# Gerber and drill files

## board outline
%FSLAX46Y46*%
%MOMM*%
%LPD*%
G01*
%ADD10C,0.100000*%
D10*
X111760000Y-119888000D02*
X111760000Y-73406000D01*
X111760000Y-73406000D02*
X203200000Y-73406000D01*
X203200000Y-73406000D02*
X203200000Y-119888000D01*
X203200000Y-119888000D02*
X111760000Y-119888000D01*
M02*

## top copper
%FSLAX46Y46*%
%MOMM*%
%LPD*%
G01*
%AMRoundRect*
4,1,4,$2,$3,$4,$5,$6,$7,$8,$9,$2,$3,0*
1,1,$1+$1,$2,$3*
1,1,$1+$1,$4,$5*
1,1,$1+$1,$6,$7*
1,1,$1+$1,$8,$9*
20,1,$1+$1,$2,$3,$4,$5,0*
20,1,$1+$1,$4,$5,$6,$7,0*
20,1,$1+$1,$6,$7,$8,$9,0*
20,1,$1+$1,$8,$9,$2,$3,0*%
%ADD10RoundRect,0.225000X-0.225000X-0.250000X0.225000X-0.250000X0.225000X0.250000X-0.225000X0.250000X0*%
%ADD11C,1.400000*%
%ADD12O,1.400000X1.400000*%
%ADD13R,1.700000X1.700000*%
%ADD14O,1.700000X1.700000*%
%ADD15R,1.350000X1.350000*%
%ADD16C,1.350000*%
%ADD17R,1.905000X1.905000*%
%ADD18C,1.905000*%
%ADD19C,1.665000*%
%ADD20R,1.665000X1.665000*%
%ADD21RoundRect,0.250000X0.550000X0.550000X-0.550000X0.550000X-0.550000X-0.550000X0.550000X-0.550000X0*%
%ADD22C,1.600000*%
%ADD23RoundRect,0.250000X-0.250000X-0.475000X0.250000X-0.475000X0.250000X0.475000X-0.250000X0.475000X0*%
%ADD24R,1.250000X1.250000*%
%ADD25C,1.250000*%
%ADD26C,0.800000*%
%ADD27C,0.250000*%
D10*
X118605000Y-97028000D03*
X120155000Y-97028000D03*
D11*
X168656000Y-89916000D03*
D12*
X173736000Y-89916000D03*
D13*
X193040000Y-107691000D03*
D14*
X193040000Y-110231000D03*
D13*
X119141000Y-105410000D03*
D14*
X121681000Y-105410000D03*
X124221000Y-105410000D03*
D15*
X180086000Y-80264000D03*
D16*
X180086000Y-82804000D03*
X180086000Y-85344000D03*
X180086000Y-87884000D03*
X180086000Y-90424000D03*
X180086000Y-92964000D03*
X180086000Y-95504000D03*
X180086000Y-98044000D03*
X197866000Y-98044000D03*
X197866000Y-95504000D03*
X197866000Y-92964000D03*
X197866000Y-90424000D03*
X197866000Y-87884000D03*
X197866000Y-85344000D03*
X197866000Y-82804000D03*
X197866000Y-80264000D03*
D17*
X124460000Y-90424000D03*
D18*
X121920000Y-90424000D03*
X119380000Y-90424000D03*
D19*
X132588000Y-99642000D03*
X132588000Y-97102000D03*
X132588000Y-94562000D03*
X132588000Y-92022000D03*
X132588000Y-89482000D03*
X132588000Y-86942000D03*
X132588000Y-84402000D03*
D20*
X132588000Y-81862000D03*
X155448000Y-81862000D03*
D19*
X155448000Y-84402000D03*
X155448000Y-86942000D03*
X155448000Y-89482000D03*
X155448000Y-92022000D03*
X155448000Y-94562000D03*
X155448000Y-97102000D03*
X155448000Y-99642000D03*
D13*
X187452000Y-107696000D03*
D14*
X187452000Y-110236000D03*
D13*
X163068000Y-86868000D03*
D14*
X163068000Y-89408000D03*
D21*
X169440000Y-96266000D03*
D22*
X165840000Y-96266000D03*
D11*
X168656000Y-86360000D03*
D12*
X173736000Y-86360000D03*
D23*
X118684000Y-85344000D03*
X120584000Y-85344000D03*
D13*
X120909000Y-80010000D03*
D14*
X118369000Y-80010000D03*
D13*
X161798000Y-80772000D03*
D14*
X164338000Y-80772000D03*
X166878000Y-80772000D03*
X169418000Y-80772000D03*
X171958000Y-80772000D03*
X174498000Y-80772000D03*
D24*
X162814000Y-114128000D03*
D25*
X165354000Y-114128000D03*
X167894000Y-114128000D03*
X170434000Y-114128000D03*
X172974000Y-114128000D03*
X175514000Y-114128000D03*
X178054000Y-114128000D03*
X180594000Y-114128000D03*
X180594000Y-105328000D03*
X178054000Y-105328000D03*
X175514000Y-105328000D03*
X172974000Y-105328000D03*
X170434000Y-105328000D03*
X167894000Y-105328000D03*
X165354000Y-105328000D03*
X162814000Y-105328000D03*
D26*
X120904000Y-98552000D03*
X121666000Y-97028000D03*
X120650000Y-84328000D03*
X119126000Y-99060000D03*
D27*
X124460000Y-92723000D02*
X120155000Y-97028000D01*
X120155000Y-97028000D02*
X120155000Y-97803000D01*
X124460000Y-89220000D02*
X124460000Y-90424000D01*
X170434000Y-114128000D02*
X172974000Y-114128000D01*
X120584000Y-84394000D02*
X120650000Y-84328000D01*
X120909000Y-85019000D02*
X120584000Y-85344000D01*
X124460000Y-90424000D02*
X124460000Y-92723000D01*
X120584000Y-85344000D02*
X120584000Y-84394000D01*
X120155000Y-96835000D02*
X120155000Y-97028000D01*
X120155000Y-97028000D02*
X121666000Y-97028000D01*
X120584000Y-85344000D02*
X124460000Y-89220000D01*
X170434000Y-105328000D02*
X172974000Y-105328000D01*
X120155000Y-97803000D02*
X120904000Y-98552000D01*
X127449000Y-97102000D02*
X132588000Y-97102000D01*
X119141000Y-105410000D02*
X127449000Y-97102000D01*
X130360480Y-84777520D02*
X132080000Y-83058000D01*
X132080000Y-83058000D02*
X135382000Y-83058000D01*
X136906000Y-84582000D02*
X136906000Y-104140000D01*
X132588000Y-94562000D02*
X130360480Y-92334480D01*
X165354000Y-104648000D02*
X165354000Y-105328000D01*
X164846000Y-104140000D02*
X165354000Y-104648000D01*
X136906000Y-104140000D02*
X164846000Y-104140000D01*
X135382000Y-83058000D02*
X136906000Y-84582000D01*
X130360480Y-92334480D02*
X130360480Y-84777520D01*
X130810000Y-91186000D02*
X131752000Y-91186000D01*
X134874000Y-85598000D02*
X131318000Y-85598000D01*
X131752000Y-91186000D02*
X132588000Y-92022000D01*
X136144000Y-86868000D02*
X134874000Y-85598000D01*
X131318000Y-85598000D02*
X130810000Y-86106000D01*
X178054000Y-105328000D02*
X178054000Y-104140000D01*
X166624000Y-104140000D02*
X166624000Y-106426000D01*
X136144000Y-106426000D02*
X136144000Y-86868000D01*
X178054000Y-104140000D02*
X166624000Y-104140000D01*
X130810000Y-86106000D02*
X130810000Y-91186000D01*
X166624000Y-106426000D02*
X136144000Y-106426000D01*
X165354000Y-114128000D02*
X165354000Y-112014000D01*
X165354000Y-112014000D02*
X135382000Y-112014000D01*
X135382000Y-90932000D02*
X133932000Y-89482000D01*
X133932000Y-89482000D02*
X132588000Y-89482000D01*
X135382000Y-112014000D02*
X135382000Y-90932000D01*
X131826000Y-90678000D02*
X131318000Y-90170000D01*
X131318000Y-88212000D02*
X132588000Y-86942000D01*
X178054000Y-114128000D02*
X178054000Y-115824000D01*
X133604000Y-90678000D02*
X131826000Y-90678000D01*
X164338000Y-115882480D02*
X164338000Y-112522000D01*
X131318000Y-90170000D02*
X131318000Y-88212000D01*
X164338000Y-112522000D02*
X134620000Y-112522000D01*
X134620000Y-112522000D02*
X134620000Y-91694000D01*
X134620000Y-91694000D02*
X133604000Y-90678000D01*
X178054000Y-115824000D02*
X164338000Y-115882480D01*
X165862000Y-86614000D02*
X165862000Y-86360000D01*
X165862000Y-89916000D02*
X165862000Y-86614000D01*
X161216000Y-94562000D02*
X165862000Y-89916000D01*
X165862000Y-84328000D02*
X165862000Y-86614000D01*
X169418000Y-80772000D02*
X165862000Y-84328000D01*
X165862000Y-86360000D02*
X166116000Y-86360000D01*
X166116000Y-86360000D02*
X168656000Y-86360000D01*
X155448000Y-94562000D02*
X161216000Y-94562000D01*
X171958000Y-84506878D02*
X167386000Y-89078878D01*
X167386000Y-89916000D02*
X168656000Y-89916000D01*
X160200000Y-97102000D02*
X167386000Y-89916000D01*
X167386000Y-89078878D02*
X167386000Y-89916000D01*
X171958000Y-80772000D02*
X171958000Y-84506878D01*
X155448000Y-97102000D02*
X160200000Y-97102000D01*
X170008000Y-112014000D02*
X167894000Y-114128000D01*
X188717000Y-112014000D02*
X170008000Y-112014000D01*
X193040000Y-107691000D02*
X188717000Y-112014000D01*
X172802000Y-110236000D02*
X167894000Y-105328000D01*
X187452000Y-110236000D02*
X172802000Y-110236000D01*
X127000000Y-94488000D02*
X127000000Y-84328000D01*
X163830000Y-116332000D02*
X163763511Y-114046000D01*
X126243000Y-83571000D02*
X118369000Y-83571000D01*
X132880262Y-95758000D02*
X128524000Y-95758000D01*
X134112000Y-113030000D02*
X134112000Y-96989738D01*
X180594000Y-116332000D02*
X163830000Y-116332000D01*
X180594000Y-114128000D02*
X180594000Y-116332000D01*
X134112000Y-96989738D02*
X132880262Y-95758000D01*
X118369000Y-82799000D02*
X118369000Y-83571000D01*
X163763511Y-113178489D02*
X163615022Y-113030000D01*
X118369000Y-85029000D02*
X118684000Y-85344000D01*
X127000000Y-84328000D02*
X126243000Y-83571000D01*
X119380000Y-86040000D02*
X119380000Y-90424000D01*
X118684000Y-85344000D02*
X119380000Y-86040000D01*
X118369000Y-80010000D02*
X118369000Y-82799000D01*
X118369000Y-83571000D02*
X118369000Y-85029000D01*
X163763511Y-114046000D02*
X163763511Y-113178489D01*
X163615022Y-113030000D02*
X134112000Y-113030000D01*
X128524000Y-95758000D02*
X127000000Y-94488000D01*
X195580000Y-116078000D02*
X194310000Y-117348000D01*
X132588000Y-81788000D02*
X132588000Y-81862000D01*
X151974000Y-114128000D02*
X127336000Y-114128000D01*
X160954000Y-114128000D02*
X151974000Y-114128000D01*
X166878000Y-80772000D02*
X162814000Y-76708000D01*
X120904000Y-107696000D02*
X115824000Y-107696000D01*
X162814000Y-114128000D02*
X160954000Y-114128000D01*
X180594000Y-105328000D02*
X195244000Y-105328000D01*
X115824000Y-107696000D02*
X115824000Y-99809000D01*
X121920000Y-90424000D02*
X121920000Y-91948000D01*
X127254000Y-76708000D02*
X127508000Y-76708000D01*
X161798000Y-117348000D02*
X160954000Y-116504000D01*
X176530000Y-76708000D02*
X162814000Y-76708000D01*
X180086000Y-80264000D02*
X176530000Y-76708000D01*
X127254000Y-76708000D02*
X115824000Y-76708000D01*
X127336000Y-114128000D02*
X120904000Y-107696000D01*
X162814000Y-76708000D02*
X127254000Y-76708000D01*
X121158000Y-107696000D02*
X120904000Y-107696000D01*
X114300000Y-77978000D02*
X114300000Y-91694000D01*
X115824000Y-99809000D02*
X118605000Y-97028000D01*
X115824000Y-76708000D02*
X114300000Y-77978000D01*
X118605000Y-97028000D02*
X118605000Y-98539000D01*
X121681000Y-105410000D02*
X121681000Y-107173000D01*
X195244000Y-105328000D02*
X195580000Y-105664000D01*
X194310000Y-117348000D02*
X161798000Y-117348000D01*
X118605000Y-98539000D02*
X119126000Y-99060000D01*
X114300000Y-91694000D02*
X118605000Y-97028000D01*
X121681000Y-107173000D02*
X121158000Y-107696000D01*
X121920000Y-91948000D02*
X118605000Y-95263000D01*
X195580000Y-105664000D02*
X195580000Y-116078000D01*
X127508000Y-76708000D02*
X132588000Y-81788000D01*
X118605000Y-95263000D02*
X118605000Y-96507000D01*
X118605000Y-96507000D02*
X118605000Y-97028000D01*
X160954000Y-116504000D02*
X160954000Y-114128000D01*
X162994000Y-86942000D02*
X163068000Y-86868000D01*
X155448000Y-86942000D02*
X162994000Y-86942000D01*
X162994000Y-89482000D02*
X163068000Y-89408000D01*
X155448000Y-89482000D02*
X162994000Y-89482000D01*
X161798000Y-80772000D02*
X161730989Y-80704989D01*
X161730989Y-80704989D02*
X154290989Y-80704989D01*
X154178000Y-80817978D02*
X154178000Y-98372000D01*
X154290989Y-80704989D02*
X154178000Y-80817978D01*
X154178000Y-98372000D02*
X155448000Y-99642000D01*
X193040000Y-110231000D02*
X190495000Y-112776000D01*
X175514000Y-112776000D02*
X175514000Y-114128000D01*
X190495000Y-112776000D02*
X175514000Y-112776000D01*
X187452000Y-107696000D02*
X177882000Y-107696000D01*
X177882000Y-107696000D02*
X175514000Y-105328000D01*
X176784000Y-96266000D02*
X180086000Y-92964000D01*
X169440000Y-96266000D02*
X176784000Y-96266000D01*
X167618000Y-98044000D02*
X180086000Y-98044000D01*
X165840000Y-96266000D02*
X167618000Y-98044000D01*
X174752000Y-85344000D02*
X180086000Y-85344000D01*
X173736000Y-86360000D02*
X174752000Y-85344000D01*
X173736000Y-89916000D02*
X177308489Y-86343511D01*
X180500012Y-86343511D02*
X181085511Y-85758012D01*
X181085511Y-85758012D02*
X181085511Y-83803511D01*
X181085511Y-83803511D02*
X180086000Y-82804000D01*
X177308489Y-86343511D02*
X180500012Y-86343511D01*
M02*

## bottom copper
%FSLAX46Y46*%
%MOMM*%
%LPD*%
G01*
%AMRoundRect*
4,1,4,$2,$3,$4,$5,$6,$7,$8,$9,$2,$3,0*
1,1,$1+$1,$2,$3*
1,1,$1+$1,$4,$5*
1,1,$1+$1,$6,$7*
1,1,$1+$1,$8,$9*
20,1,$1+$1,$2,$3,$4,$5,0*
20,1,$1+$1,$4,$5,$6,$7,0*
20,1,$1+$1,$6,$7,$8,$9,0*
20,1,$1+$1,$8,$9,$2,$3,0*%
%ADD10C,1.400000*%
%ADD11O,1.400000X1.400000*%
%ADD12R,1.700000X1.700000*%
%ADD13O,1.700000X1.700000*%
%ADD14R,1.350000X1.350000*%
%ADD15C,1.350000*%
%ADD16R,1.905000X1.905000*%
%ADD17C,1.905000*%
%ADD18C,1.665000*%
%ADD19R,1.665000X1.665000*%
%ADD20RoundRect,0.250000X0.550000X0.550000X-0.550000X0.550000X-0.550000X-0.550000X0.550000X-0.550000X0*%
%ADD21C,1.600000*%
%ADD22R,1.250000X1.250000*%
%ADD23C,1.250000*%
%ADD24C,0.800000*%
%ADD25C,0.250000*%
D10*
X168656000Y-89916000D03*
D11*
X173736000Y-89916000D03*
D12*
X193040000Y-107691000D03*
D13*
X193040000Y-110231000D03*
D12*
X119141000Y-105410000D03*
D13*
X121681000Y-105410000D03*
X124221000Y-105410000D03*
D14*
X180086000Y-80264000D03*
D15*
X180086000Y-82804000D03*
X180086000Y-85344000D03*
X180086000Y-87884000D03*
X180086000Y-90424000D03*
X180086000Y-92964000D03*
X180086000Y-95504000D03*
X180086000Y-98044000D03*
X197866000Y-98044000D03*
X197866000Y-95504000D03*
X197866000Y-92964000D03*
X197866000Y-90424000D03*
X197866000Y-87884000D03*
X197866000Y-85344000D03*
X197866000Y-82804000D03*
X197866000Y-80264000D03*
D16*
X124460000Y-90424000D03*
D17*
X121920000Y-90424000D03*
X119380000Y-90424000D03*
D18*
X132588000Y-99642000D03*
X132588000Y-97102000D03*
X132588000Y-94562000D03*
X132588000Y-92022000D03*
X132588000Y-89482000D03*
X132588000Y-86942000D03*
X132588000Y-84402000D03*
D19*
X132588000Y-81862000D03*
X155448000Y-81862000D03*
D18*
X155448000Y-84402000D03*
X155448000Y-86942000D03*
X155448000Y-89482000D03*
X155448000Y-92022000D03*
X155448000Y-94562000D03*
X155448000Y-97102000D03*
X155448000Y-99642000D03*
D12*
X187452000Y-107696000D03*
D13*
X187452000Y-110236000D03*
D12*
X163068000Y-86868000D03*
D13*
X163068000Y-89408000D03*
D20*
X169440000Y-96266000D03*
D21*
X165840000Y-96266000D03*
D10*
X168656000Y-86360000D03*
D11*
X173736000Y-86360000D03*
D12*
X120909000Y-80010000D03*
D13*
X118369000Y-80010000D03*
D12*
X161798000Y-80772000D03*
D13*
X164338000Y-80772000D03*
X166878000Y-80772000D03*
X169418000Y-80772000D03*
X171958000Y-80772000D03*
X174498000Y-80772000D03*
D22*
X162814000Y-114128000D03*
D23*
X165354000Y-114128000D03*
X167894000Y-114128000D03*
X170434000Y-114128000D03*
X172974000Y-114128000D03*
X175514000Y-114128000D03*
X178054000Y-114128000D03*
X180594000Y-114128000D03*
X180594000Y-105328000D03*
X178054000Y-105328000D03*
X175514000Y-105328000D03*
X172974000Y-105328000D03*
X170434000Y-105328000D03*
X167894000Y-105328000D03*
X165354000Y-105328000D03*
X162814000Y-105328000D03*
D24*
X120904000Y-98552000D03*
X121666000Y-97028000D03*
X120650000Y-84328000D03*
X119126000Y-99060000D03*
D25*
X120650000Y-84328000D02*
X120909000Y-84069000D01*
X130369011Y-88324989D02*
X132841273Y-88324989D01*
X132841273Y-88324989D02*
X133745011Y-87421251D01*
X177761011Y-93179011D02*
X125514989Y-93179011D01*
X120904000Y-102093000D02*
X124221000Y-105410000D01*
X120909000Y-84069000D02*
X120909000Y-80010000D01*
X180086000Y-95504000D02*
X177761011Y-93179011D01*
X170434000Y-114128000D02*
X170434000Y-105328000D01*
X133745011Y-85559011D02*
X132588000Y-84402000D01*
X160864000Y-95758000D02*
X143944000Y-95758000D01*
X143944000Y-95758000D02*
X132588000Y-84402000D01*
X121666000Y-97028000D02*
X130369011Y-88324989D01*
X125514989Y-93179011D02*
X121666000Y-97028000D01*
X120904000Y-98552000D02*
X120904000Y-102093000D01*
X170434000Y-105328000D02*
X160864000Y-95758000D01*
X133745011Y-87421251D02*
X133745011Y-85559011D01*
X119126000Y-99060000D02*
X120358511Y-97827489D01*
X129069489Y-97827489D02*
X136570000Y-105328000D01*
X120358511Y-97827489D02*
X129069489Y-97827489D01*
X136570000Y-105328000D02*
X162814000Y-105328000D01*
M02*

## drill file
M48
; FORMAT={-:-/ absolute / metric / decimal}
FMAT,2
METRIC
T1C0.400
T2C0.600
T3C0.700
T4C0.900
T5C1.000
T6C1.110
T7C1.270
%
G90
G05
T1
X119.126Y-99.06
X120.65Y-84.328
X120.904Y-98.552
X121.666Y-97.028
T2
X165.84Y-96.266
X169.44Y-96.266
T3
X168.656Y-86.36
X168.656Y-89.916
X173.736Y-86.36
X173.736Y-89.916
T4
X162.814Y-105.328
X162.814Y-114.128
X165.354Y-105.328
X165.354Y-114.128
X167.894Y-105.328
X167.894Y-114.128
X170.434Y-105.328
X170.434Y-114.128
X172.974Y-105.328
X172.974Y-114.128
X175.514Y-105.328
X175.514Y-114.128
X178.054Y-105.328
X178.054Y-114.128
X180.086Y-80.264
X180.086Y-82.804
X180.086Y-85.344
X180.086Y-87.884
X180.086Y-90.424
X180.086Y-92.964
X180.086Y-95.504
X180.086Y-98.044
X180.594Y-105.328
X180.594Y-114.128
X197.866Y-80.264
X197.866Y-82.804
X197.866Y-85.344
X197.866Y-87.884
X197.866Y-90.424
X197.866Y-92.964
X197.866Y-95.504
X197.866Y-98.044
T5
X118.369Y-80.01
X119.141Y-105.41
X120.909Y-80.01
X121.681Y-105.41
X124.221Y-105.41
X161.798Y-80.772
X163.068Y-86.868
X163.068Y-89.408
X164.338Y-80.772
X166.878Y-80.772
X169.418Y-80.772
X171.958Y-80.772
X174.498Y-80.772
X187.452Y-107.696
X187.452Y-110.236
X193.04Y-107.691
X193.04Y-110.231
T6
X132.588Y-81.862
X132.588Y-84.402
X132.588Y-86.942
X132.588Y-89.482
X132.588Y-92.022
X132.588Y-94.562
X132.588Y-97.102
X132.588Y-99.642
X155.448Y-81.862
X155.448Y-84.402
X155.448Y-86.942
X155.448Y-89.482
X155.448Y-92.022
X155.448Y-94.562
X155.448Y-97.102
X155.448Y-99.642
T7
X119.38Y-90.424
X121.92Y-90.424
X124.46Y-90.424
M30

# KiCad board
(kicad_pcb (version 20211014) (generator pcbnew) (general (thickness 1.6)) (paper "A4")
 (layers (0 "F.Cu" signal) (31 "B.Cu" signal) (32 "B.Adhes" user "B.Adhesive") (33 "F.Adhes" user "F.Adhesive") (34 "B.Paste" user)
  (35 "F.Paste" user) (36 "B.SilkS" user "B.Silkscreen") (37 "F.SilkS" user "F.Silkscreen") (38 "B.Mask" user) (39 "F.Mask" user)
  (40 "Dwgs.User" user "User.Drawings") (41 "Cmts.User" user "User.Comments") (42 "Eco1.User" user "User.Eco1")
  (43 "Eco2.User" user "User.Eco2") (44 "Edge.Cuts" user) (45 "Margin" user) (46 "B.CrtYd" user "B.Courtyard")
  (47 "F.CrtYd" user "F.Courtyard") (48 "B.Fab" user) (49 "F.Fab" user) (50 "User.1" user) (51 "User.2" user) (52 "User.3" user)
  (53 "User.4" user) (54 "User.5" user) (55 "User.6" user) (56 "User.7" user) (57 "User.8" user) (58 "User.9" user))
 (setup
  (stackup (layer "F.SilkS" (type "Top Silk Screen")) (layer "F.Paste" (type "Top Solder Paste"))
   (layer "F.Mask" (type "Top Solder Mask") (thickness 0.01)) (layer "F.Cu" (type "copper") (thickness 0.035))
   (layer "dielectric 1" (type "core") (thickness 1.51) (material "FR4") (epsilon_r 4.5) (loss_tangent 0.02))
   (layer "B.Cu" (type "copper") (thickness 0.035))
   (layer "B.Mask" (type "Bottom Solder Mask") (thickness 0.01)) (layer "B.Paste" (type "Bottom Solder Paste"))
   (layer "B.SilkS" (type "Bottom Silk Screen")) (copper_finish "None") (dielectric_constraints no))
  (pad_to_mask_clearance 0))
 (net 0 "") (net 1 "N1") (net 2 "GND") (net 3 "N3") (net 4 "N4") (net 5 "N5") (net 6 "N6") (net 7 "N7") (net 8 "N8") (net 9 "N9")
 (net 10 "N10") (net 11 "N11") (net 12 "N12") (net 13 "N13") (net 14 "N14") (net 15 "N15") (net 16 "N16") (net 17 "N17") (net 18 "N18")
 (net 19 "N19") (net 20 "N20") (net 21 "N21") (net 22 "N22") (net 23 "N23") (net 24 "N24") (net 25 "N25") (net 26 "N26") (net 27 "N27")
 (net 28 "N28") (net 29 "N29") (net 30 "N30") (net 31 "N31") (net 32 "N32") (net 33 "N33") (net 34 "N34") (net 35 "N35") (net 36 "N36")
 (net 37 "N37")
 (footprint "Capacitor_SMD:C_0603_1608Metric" (layer "F.Cu") (at 119.38 97.028)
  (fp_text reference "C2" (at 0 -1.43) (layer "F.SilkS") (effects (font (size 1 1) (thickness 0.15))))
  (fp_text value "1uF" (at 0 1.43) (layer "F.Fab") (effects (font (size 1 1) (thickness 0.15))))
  (pad "1" smd roundrect locked (at -0.775 0) (size 0.9 0.95) (layers "F.Cu" "F.Paste" "F.Mask") (roundrect_rratio 0.25) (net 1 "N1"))
  (pad "2" smd roundrect locked (at 0.775 0) (size 0.9 0.95) (layers "F.Cu" "F.Paste" "F.Mask") (roundrect_rratio 0.25) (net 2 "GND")))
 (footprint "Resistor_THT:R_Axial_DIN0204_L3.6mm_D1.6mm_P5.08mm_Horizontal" (layer "F.Cu") (at 168.656 89.916)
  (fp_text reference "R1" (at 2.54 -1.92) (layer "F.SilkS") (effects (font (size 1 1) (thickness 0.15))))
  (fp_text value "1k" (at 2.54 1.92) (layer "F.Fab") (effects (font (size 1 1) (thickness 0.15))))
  (pad "1" thru_hole circle locked (at 0 0) (size 1.4 1.4) (drill 0.7) (layers *.Cu *.Mask) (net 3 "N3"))
  (pad "2" thru_hole oval locked (at 5.08 0) (size 1.4 1.4) (drill 0.7) (layers *.Cu *.Mask) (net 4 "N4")))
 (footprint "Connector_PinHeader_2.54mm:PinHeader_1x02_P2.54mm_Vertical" (layer "F.Cu") (at 193.04 107.691)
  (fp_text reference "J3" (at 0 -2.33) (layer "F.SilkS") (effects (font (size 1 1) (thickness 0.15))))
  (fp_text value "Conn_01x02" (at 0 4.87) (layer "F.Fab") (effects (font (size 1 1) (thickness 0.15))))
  (pad "1" thru_hole rect locked (at 0 0) (size 1.7 1.7) (drill 1) (layers *.Cu *.Mask) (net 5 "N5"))
  (pad "2" thru_hole oval locked (at 0 2.54) (size 1.7 1.7) (drill 1) (layers *.Cu *.Mask) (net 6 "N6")))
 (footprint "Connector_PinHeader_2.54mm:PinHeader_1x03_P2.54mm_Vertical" (layer "F.Cu") (at 119.141 105.41 90)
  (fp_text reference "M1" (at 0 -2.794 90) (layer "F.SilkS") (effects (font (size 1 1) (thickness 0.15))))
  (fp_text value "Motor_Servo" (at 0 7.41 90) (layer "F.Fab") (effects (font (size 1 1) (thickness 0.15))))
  (pad "1" thru_hole rect locked (at 0 0 90) (size 1.7 1.7) (drill 1) (layers *.Cu *.Mask) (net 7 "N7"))
  (pad "2" thru_hole oval locked (at 0 2.54 90) (size 1.7 1.7) (drill 1) (layers *.Cu *.Mask) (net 1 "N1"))
  (pad "3" thru_hole oval locked (at 0 5.08 90) (size 1.7 1.7) (drill 1) (layers *.Cu *.Mask) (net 2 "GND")))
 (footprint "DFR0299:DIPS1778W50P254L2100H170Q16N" (layer "F.Cu") (at 180.086 80.264)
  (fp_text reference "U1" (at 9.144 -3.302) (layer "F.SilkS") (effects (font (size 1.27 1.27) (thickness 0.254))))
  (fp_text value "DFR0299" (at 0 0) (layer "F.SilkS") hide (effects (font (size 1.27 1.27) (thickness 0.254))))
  (pad "1" thru_hole rect locked (at 0 0) (size 1.35 1.35) (drill 0.9) (layers *.Cu *.Mask) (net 1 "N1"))
  (pad "2" thru_hole circle locked (at 0 2.54) (size 1.35 1.35) (drill 0.9) (layers *.Cu *.Mask) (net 4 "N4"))
  (pad "3" thru_hole circle locked (at 0 5.08) (size 1.35 1.35) (drill 0.9) (layers *.Cu *.Mask) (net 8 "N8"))
  (pad "4" thru_hole circle locked (at 0 7.62) (size 1.35 1.35) (drill 0.9) (layers *.Cu *.Mask) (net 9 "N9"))
  (pad "5" thru_hole circle locked (at 0 10.16) (size 1.35 1.35) (drill 0.9) (layers *.Cu *.Mask) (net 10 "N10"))
  (pad "6" thru_hole circle locked (at 0 12.7) (size 1.35 1.35) (drill 0.9) (layers *.Cu *.Mask) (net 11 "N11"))
  (pad "7" thru_hole circle locked (at 0 15.24) (size 1.35 1.35) (drill 0.9) (layers *.Cu *.Mask) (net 2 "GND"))
  (pad "8" thru_hole circle locked (at 0 17.78) (size 1.35 1.35) (drill 0.9) (layers *.Cu *.Mask) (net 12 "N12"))
  (pad "9" thru_hole circle locked (at 17.78 17.78) (size 1.35 1.35) (drill 0.9) (layers *.Cu *.Mask) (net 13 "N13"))
  (pad "10" thru_hole circle locked (at 17.78 15.24) (size 1.35 1.35) (drill 0.9) (layers *.Cu *.Mask) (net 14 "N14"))
  (pad "11" thru_hole circle locked (at 17.78 12.7) (size 1.35 1.35) (drill 0.9) (layers *.Cu *.Mask) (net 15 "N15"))
  (pad "12" thru_hole circle locked (at 17.78 10.16) (size 1.35 1.35) (drill 0.9) (layers *.Cu *.Mask) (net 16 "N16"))
  (pad "13" thru_hole circle locked (at 17.78 7.62) (size 1.35 1.35) (drill 0.9) (layers *.Cu *.Mask) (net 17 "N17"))
  (pad "14" thru_hole circle locked (at 17.78 5.08) (size 1.35 1.35) (drill 0.9) (layers *.Cu *.Mask) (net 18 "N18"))
  (pad "15" thru_hole circle locked (at 17.78 2.54) (size 1.35 1.35) (drill 0.9) (layers *.Cu *.Mask) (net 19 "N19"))
  (pad "16" thru_hole circle locked (at 17.78 0) (size 1.35 1.35) (drill 0.9) (layers *.Cu *.Mask) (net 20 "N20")))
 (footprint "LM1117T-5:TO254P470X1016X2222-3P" (layer "F.Cu") (at 119.38 91.44 180)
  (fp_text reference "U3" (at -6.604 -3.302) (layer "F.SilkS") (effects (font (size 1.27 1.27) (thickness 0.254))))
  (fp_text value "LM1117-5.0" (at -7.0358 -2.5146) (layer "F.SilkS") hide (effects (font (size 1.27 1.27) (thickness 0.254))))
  (pad "1" thru_hole rect locked (at -5.08 1.016 180) (size 1.905 1.905) (drill 1.27) (layers *.Cu *.Mask) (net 2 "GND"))
  (pad "2" thru_hole circle locked (at -2.54 1.016 180) (size 1.905 1.905) (drill 1.27) (layers *.Cu *.Mask) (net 1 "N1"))
  (pad "3" thru_hole circle locked (at 0 1.016 180) (size 1.905 1.905) (drill 1.27) (layers *.Cu *.Mask) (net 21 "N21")))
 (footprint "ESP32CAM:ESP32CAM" (layer "F.Cu") (at 132.588 99.642)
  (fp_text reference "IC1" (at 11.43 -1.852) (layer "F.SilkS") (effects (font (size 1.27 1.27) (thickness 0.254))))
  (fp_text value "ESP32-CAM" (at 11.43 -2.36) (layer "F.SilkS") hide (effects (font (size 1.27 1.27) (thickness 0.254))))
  (pad "1" thru_hole circle locked (at 0 0) (size 1.665 1.665) (drill 1.11) (layers *.Cu *.Mask) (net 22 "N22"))
  (pad "2" thru_hole circle locked (at 0 -2.54) (size 1.665 1.665) (drill 1.11) (layers *.Cu *.Mask) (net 7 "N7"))
  (pad "3" thru_hole circle locked (at 0 -5.08) (size 1.665 1.665) (drill 1.11) (layers *.Cu *.Mask) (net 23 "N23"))
  (pad "4" thru_hole circle locked (at 0 -7.62) (size 1.665 1.665) (drill 1.11) (layers *.Cu *.Mask) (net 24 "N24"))
  (pad "5" thru_hole circle locked (at 0 -10.16) (size 1.665 1.665) (drill 1.11) (layers *.Cu *.Mask) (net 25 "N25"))
  (pad "6" thru_hole circle locked (at 0 -12.7) (size 1.665 1.665) (drill 1.11) (layers *.Cu *.Mask) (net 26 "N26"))
  (pad "7" thru_hole circle locked (at 0 -15.24) (size 1.665 1.665) (drill 1.11) (layers *.Cu *.Mask) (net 2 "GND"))
  (pad "8" thru_hole rect locked (at 0 -17.78) (size 1.665 1.665) (drill 1.11) (layers *.Cu *.Mask) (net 1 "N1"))
  (pad "9" thru_hole rect locked (at 22.86 -17.78) (size 1.665 1.665) (drill 1.11) (layers *.Cu *.Mask) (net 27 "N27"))
  (pad "10" thru_hole circle locked (at 22.86 -15.24) (size 1.665 1.665) (drill 1.11) (layers *.Cu *.Mask) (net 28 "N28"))
  (pad "11" thru_hole circle locked (at 22.86 -12.7) (size 1.665 1.665) (drill 1.11) (layers *.Cu *.Mask) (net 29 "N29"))
  (pad "12" thru_hole circle locked (at 22.86 -10.16) (size 1.665 1.665) (drill 1.11) (layers *.Cu *.Mask) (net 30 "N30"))
  (pad "13" thru_hole circle locked (at 22.86 -7.62) (size 1.665 1.665) (drill 1.11) (layers *.Cu *.Mask) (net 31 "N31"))
  (pad "14" thru_hole circle locked (at 22.86 -5.08) (size 1.665 1.665) (drill 1.11) (layers *.Cu *.Mask) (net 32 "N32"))
  (pad "15" thru_hole circle locked (at 22.86 -2.54) (size 1.665 1.665) (drill 1.11) (layers *.Cu *.Mask) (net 3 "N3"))
  (pad "16" thru_hole circle locked (at 22.86 0) (size 1.665 1.665) (drill 1.11) (layers *.Cu *.Mask) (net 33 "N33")))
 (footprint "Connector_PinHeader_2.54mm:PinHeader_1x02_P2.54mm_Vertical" (layer "F.Cu") (at 187.452 107.696)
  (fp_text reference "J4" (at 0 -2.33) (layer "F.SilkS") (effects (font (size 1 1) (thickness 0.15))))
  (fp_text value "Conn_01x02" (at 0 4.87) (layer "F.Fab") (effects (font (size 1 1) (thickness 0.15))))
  (pad "1" thru_hole rect locked (at 0 0) (size 1.7 1.7) (drill 1) (layers *.Cu *.Mask) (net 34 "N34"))
  (pad "2" thru_hole oval locked (at 0 2.54) (size 1.7 1.7) (drill 1) (layers *.Cu *.Mask) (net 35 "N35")))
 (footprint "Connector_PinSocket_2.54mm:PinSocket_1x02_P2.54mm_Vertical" (layer "F.Cu") (at 163.068 86.868)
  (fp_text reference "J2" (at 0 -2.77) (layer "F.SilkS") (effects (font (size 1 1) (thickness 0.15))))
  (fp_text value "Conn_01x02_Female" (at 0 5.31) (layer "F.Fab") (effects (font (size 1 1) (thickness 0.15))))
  (pad "1" thru_hole rect locked (at 0 0) (size 1.7 1.7) (drill 1) (layers *.Cu *.Mask) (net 29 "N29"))
  (pad "2" thru_hole oval locked (at 0 2.54) (size 1.7 1.7) (drill 1) (layers *.Cu *.Mask) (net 30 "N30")))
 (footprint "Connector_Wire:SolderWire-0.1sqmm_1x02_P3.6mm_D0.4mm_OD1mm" (layer "F.Cu") (at 169.44 96.266 180)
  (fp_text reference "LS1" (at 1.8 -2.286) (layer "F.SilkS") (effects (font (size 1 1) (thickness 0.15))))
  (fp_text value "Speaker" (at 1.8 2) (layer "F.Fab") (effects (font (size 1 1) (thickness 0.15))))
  (pad "1" thru_hole roundrect locked (at 0 0 180) (size 1.6 1.6) (drill 0.6) (layers *.Cu *.Mask) (roundrect_rratio 0.15625) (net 11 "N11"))
  (pad "2" thru_hole circle locked (at 3.6 0 180) (size 1.6 1.6) (drill 0.6) (layers *.Cu *.Mask) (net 12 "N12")))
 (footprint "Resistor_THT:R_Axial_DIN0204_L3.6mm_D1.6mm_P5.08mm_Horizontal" (layer "F.Cu") (at 168.656 86.36)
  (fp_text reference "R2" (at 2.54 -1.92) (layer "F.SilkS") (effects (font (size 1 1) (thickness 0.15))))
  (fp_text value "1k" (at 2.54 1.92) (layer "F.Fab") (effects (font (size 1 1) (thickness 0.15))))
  (pad "1" thru_hole circle locked (at 0 0) (size 1.4 1.4) (drill 0.7) (layers *.Cu *.Mask) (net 32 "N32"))
  (pad "2" thru_hole oval locked (at 5.08 0) (size 1.4 1.4) (drill 0.7) (layers *.Cu *.Mask) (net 8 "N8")))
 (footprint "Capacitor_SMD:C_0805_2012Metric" (layer "F.Cu") (at 119.634 85.344)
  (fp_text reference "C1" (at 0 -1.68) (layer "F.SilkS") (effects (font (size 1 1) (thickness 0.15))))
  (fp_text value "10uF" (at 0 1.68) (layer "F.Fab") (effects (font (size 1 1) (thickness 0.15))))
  (pad "1" smd roundrect locked (at -0.95 0) (size 1 1.45) (layers "F.Cu" "F.Paste" "F.Mask") (roundrect_rratio 0.25) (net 21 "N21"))
  (pad "2" smd roundrect locked (at 0.95 0) (size 1 1.45) (layers "F.Cu" "F.Paste" "F.Mask") (roundrect_rratio 0.25) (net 2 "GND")))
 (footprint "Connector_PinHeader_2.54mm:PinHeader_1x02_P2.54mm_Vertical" (layer "F.Cu") (at 120.909 80.01 -90)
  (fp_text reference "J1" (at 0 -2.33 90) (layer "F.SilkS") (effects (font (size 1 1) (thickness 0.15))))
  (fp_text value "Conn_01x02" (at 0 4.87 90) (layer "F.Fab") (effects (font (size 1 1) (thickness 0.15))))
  (pad "1" thru_hole rect locked (at 0 0 270) (size 1.7 1.7) (drill 1) (layers *.Cu *.Mask) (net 2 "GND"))
  (pad "2" thru_hole oval locked (at 0 2.54 270) (size 1.7 1.7) (drill 1) (layers *.Cu *.Mask) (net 21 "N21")))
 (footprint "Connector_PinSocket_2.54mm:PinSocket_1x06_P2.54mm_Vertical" (layer "F.Cu") (at 161.798 80.772 90)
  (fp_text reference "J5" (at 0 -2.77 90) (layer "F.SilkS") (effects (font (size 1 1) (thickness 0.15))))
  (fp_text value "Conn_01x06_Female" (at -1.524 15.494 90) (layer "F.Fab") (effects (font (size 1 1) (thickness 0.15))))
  (pad "1" thru_hole rect locked (at 0 0 90) (size 1.7 1.7) (drill 1) (layers *.Cu *.Mask) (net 33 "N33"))
  (pad "2" thru_hole oval locked (at 0 2.54 90) (size 1.7 1.7) (drill 1) (layers *.Cu *.Mask) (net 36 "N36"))
  (pad "3" thru_hole oval locked (at 0 5.08 90) (size 1.7 1.7) (drill 1) (layers *.Cu *.Mask) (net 1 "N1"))
  (pad "4" thru_hole oval locked (at 0 7.62 90) (size 1.7 1.7) (drill 1) (layers *.Cu *.Mask) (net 32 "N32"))
  (pad "5" thru_hole oval locked (at 0 10.16 90) (size 1.7 1.7) (drill 1) (layers *.Cu *.Mask) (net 3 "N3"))
  (pad "6" thru_hole oval locked (at 0 12.7 90) (size 1.7 1.7) (drill 1) (layers *.Cu *.Mask) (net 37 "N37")))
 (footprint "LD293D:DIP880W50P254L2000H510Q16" (layer "F.Cu") (at 171.704 109.728 90)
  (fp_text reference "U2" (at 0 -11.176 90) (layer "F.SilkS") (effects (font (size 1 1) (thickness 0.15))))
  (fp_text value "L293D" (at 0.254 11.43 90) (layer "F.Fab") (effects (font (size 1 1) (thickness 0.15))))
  (pad "1" thru_hole rect locked (at -4.4 -8.89 90) (size 1.25 1.25) (drill 0.9) (layers *.Cu *.Mask) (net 1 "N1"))
  (pad "2" thru_hole circle locked (at -4.4 -6.35 90) (size 1.25 1.25) (drill 0.9) (layers *.Cu *.Mask) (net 25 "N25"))
  (pad "3" thru_hole circle locked (at -4.4 -3.81 90) (size 1.25 1.25) (drill 0.9) (layers *.Cu *.Mask) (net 5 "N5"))
  (pad "4" thru_hole circle locked (at -4.4 -1.27 90) (size 1.25 1.25) (drill 0.9) (layers *.Cu *.Mask) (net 2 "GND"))
  (pad "5" thru_hole circle locked (at -4.4 1.27 90) (size 1.25 1.25) (drill 0.9) (layers *.Cu *.Mask) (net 2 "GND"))
  (pad "6" thru_hole circle locked (at -4.4 3.81 90) (size 1.25 1.25) (drill 0.9) (layers *.Cu *.Mask) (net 6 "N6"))
  (pad "7" thru_hole circle locked (at -4.4 6.35 90) (size 1.25 1.25) (drill 0.9) (layers *.Cu *.Mask) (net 26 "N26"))
  (pad "8" thru_hole circle locked (at -4.4 8.89 90) (size 1.25 1.25) (drill 0.9) (layers *.Cu *.Mask) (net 21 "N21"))
  (pad "9" thru_hole circle locked (at 4.4 8.89 90) (size 1.25 1.25) (drill 0.9) (layers *.Cu *.Mask) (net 1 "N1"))
  (pad "10" thru_hole circle locked (at 4.4 6.35 90) (size 1.25 1.25) (drill 0.9) (layers *.Cu *.Mask) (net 24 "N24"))
  (pad "11" thru_hole circle locked (at 4.4 3.81 90) (size 1.25 1.25) (drill 0.9) (layers *.Cu *.Mask) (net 34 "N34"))
  (pad "12" thru_hole circle locked (at 4.4 1.27 90) (size 1.25 1.25) (drill 0.9) (layers *.Cu *.Mask) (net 2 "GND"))
  (pad "13" thru_hole circle locked (at 4.4 -1.27 90) (size 1.25 1.25) (drill 0.9) (layers *.Cu *.Mask) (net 2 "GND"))
  (pad "14" thru_hole circle locked (at 4.4 -3.81 90) (size 1.25 1.25) (drill 0.9) (layers *.Cu *.Mask) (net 35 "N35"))
  (pad "15" thru_hole circle locked (at 4.4 -6.35 90) (size 1.25 1.25) (drill 0.9) (layers *.Cu *.Mask) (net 23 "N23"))
  (pad "16" thru_hole circle locked (at 4.4 -8.89 90) (size 1.25 1.25) (drill 0.9) (layers *.Cu *.Mask) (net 1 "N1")))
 (gr_line (start 111.76 119.888) (end 111.76 73.406) (layer "Edge.Cuts") (width 0.1))
 (gr_line (start 111.76 73.406) (end 203.2 73.406) (layer "Edge.Cuts") (width 0.1))
 (gr_line (start 203.2 73.406) (end 203.2 119.888) (layer "Edge.Cuts") (width 0.1))
 (gr_line (start 203.2 119.888) (end 111.76 119.888) (layer "Edge.Cuts") (width 0.1))
 (segment (start 124.46 92.723) (end 120.155 97.028) (width 0.25) (layer "F.Cu") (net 2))
 (segment (start 120.155 97.028) (end 120.155 97.803) (width 0.25) (layer "F.Cu") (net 2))
 (segment (start 124.46 89.22) (end 124.46 90.424) (width 0.25) (layer "F.Cu") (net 2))
 (segment (start 170.434 114.128) (end 172.974 114.128) (width 0.25) (layer "F.Cu") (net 2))
 (segment (start 120.584 84.394) (end 120.65 84.328) (width 0.25) (layer "F.Cu") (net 2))
 (segment (start 120.909 85.019) (end 120.584 85.344) (width 0.25) (layer "F.Cu") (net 2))
 (segment (start 124.46 90.424) (end 124.46 92.723) (width 0.25) (layer "F.Cu") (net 2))
 (segment (start 120.584 85.344) (end 120.584 84.394) (width 0.25) (layer "F.Cu") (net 2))
 (segment (start 120.155 96.835) (end 120.155 97.028) (width 0.25) (layer "F.Cu") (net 2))
 (segment (start 120.155 97.028) (end 121.666 97.028) (width 0.25) (layer "F.Cu") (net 2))
 (segment (start 120.584 85.344) (end 124.46 89.22) (width 0.25) (layer "F.Cu") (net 2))
 (segment (start 170.434 105.328) (end 172.974 105.328) (width 0.25) (layer "F.Cu") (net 2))
 (segment (start 120.155 97.803) (end 120.904 98.552) (width 0.25) (layer "F.Cu") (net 2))
 (via (at 120.904 98.552) (size 0.8) (drill 0.4) (layers "F.Cu" "B.Cu") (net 2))
 (via (at 121.666 97.028) (size 0.8) (drill 0.4) (layers "F.Cu" "B.Cu") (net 2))
 (via (at 120.65 84.328) (size 0.8) (drill 0.4) (layers "F.Cu" "B.Cu") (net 2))
 (segment (start 120.65 84.328) (end 120.909 84.069) (width 0.25) (layer "B.Cu") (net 2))
 (segment (start 130.369011 88.324989) (end 132.841273 88.324989) (width 0.25) (layer "B.Cu") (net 2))
 (segment (start 132.841273 88.324989) (end 133.745011 87.421251) (width 0.25) (layer "B.Cu") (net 2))
 (segment (start 177.761011 93.179011) (end 125.514989 93.179011) (width 0.25) (layer "B.Cu") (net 2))
 (segment (start 120.904 102.093) (end 124.221 105.41) (width 0.25) (layer "B.Cu") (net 2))
 (segment (start 120.909 84.069) (end 120.909 80.01) (width 0.25) (layer "B.Cu") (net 2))
 (segment (start 180.086 95.504) (end 177.761011 93.179011) (width 0.25) (layer "B.Cu") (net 2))
 (segment (start 170.434 114.128) (end 170.434 105.328) (width 0.25) (layer "B.Cu") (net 2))
 (segment (start 133.745011 85.559011) (end 132.588 84.402) (width 0.25) (layer "B.Cu") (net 2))
 (segment (start 160.864 95.758) (end 143.944 95.758) (width 0.25) (layer "B.Cu") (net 2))
 (segment (start 143.944 95.758) (end 132.588 84.402) (width 0.25) (layer "B.Cu") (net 2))
 (segment (start 121.666 97.028) (end 130.369011 88.324989) (width 0.25) (layer "B.Cu") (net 2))
 (segment (start 125.514989 93.179011) (end 121.666 97.028) (width 0.25) (layer "B.Cu") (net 2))
 (segment (start 120.904 98.552) (end 120.904 102.093) (width 0.25) (layer "B.Cu") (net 2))
 (segment (start 170.434 105.328) (end 160.864 95.758) (width 0.25) (layer "B.Cu") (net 2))
 (segment (start 133.745011 87.421251) (end 133.745011 85.559011) (width 0.25) (layer "B.Cu") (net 2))
 (segment (start 127.449 97.102) (end 132.588 97.102) (width 0.25) (layer "F.Cu") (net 7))
 (segment (start 119.141 105.41) (end 127.449 97.102) (width 0.25) (layer "F.Cu") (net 7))
 (segment (start 130.36048 84.77752) (end 132.08 83.058) (width 0.25) (layer "F.Cu") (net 23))
 (segment (start 132.08 83.058) (end 135.382 83.058) (width 0.25) (layer "F.Cu") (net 23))
 (segment (start 136.906 84.582) (end 136.906 104.14) (width 0.25) (layer "F.Cu") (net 23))
 (segment (start 132.588 94.562) (end 130.36048 92.33448) (width 0.25) (layer "F.Cu") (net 23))
 (segment (start 165.354 104.648) (end 165.354 105.328) (width 0.25) (layer "F.Cu") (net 23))
 (segment (start 164.846 104.14) (end 165.354 104.648) (width 0.25) (layer "F.Cu") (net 23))
 (segment (start 136.906 104.14) (end 164.846 104.14) (width 0.25) (layer "F.Cu") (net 23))
 (segment (start 135.382 83.058) (end 136.906 84.582) (width 0.25) (layer "F.Cu") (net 23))
 (segment (start 130.36048 92.33448) (end 130.36048 84.77752) (width 0.25) (layer "F.Cu") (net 23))
 (segment (start 130.81 91.186) (end 131.752 91.186) (width 0.25) (layer "F.Cu") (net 24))
 (segment (start 134.874 85.598) (end 131.318 85.598) (width 0.25) (layer "F.Cu") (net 24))
 (segment (start 131.752 91.186) (end 132.588 92.022) (width 0.25) (layer "F.Cu") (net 24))
 (segment (start 136.144 86.868) (end 134.874 85.598) (width 0.25) (layer "F.Cu") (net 24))
 (segment (start 131.318 85.598) (end 130.81 86.106) (width 0.25) (layer "F.Cu") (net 24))
 (segment (start 178.054 105.328) (end 178.054 104.14) (width 0.25) (layer "F.Cu") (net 24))
 (segment (start 166.624 104.14) (end 166.624 106.426) (width 0.25) (layer "F.Cu") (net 24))
 (segment (start 136.144 106.426) (end 136.144 86.868) (width 0.25) (layer "F.Cu") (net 24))
 (segment (start 178.054 104.14) (end 166.624 104.14) (width 0.25) (layer "F.Cu") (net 24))
 (segment (start 130.81 86.106) (end 130.81 91.186) (width 0.25) (layer "F.Cu") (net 24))
 (segment (start 166.624 106.426) (end 136.144 106.426) (width 0.25) (layer "F.Cu") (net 24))
 (segment (start 165.354 114.128) (end 165.354 112.014) (width 0.25) (layer "F.Cu") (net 25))
 (segment (start 165.354 112.014) (end 135.382 112.014) (width 0.25) (layer "F.Cu") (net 25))
 (segment (start 135.382 90.932) (end 133.932 89.482) (width 0.25) (layer "F.Cu") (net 25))
 (segment (start 133.932 89.482) (end 132.588 89.482) (width 0.25) (layer "F.Cu") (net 25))
 (segment (start 135.382 112.014) (end 135.382 90.932) (width 0.25) (layer "F.Cu") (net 25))
 (segment (start 131.826 90.678) (end 131.318 90.17) (width 0.25) (layer "F.Cu") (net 26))
 (segment (start 131.318 88.212) (end 132.588 86.942) (width 0.25) (layer "F.Cu") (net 26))
 (segment (start 178.054 114.128) (end 178.054 115.824) (width 0.25) (layer "F.Cu") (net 26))
 (segment (start 133.604 90.678) (end 131.826 90.678) (width 0.25) (layer "F.Cu") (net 26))
 (segment (start 164.338 115.88248) (end 164.338 112.522) (width 0.25) (layer "F.Cu") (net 26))
 (segment (start 131.318 90.17) (end 131.318 88.212) (width 0.25) (layer "F.Cu") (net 26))
 (segment (start 164.338 112.522) (end 134.62 112.522) (width 0.25) (layer "F.Cu") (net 26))
 (segment (start 134.62 112.522) (end 134.62 91.694) (width 0.25) (layer "F.Cu") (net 26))
 (segment (start 134.62 91.694) (end 133.604 90.678) (width 0.25) (layer "F.Cu") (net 26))
 (segment (start 178.054 115.824) (end 164.338 115.88248) (width 0.25) (layer "F.Cu") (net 26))
 (segment (start 165.862 86.614) (end 165.862 86.36) (width 0.25) (layer "F.Cu") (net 32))
 (segment (start 165.862 89.916) (end 165.862 86.614) (width 0.25) (layer "F.Cu") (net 32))
 (segment (start 161.216 94.562) (end 165.862 89.916) (width 0.25) (layer "F.Cu") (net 32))
 (segment (start 165.862 84.328) (end 165.862 86.614) (width 0.25) (layer "F.Cu") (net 32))
 (segment (start 169.418 80.772) (end 165.862 84.328) (width 0.25) (layer "F.Cu") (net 32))
 (segment (start 165.862 86.36) (end 166.116 86.36) (width 0.25) (layer "F.Cu") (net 32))
 (segment (start 166.116 86.36) (end 168.656 86.36) (width 0.25) (layer "F.Cu") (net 32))
 (segment (start 155.448 94.562) (end 161.216 94.562) (width 0.25) (layer "F.Cu") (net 32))
 (segment (start 171.958 84.506878) (end 167.386 89.078878) (width 0.25) (layer "F.Cu") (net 3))
 (segment (start 167.386 89.916) (end 168.656 89.916) (width 0.25) (layer "F.Cu") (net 3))
 (segment (start 160.2 97.102) (end 167.386 89.916) (width 0.25) (layer "F.Cu") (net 3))
 (segment (start 167.386 89.078878) (end 167.386 89.916) (width 0.25) (layer "F.Cu") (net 3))
 (segment (start 171.958 80.772) (end 171.958 84.506878) (width 0.25) (layer "F.Cu") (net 3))
 (segment (start 155.448 97.102) (end 160.2 97.102) (width 0.25) (layer "F.Cu") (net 3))
 (segment (start 170.008 112.014) (end 167.894 114.128) (width 0.25) (layer "F.Cu") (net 5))
 (segment (start 188.717 112.014) (end 170.008 112.014) (width 0.25) (layer "F.Cu") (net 5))
 (segment (start 193.04 107.691) (end 188.717 112.014) (width 0.25) (layer "F.Cu") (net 5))
 (segment (start 172.802 110.236) (end 167.894 105.328) (width 0.25) (layer "F.Cu") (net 35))
 (segment (start 187.452 110.236) (end 172.802 110.236) (width 0.25) (layer "F.Cu") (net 35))
 (segment (start 127 94.488) (end 127 84.328) (width 0.25) (layer "F.Cu") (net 21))
 (segment (start 163.83 116.332) (end 163.763511 114.046) (width 0.25) (layer "F.Cu") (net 21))
 (segment (start 126.243 83.571) (end 118.369 83.571) (width 0.25) (layer "F.Cu") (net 21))
 (segment (start 132.880262 95.758) (end 128.524 95.758) (width 0.25) (layer "F.Cu") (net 21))
 (segment (start 134.112 113.03) (end 134.112 96.989738) (width 0.25) (layer "F.Cu") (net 21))
 (segment (start 180.594 116.332) (end 163.83 116.332) (width 0.25) (layer "F.Cu") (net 21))
 (segment (start 180.594 114.128) (end 180.594 116.332) (width 0.25) (layer "F.Cu") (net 21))
 (segment (start 134.112 96.989738) (end 132.880262 95.758) (width 0.25) (layer "F.Cu") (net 21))
 (segment (start 118.369 82.799) (end 118.369 83.571) (width 0.25) (layer "F.Cu") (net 21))
 (segment (start 163.763511 113.178489) (end 163.615022 113.03) (width 0.25) (layer "F.Cu") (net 21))
 (segment (start 118.369 85.029) (end 118.684 85.344) (width 0.25) (layer "F.Cu") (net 21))
 (segment (start 127 84.328) (end 126.243 83.571) (width 0.25) (layer "F.Cu") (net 21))
 (segment (start 119.38 86.04) (end 119.38 90.424) (width 0.25) (layer "F.Cu") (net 21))
 (segment (start 118.684 85.344) (end 119.38 86.04) (width 0.25) (layer "F.Cu") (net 21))
 (segment (start 118.369 80.01) (end 118.369 82.799) (width 0.25) (layer "F.Cu") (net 21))
 (segment (start 118.369 83.571) (end 118.369 85.029) (width 0.25) (layer "F.Cu") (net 21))
 (segment (start 163.763511 114.046) (end 163.763511 113.178489) (width 0.25) (layer "F.Cu") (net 21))
 (segment (start 163.615022 113.03) (end 134.112 113.03) (width 0.25) (layer "F.Cu") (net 21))
 (segment (start 128.524 95.758) (end 127 94.488) (width 0.25) (layer "F.Cu") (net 21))
 (segment (start 195.58 116.078) (end 194.31 117.348) (width 0.25) (layer "F.Cu") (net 1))
 (segment (start 132.588 81.788) (end 132.588 81.862) (width 0.25) (layer "F.Cu") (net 1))
 (segment (start 151.974 114.128) (end 127.336 114.128) (width 0.25) (layer "F.Cu") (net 1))
 (segment (start 160.954 114.128) (end 151.974 114.128) (width 0.25) (layer "F.Cu") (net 1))
 (segment (start 166.878 80.772) (end 162.814 76.708) (width 0.25) (layer "F.Cu") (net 1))
 (segment (start 120.904 107.696) (end 115.824 107.696) (width 0.25) (layer "F.Cu") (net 1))
 (segment (start 162.814 114.128) (end 160.954 114.128) (width 0.25) (layer "F.Cu") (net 1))
 (segment (start 180.594 105.328) (end 195.244 105.328) (width 0.25) (layer "F.Cu") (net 1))
 (segment (start 115.824 107.696) (end 115.824 99.809) (width 0.25) (layer "F.Cu") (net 1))
 (segment (start 121.92 90.424) (end 121.92 91.948) (width 0.25) (layer "F.Cu") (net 1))
 (segment (start 127.254 76.708) (end 127.508 76.708) (width 0.25) (layer "F.Cu") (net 1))
 (segment (start 161.798 117.348) (end 160.954 116.504) (width 0.25) (layer "F.Cu") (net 1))
 (segment (start 176.53 76.708) (end 162.814 76.708) (width 0.25) (layer "F.Cu") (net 1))
 (segment (start 180.086 80.264) (end 176.53 76.708) (width 0.25) (layer "F.Cu") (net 1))
 (segment (start 127.254 76.708) (end 115.824 76.708) (width 0.25) (layer "F.Cu") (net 1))
 (segment (start 127.336 114.128) (end 120.904 107.696) (width 0.25) (layer "F.Cu") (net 1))
 (segment (start 162.814 76.708) (end 127.254 76.708) (width 0.25) (layer "F.Cu") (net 1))
 (segment (start 121.158 107.696) (end 120.904 107.696) (width 0.25) (layer "F.Cu") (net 1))
 (segment (start 114.3 77.978) (end 114.3 91.694) (width 0.25) (layer "F.Cu") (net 1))
 (segment (start 115.824 99.809) (end 118.605 97.028) (width 0.25) (layer "F.Cu") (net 1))
 (segment (start 115.824 76.708) (end 114.3 77.978) (width 0.25) (layer "F.Cu") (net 1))
 (segment (start 118.605 97.028) (end 118.605 98.539) (width 0.25) (layer "F.Cu") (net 1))
 (segment (start 121.681 105.41) (end 121.681 107.173) (width 0.25) (layer "F.Cu") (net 1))
 (segment (start 195.244 105.328) (end 195.58 105.664) (width 0.25) (layer "F.Cu") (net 1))
 (segment (start 194.31 117.348) (end 161.798 117.348) (width 0.25) (layer "F.Cu") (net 1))
 (segment (start 118.605 98.539) (end 119.126 99.06) (width 0.25) (layer "F.Cu") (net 1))
 (segment (start 114.3 91.694) (end 118.605 97.028) (width 0.25) (layer "F.Cu") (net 1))
 (segment (start 121.681 107.173) (end 121.158 107.696) (width 0.25) (layer "F.Cu") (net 1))
 (segment (start 121.92 91.948) (end 118.605 95.263) (width 0.25) (layer "F.Cu") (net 1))
 (segment (start 195.58 105.664) (end 195.58 116.078) (width 0.25) (layer "F.Cu") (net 1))
 (segment (start 127.508 76.708) (end 132.588 81.788) (width 0.25) (layer "F.Cu") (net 1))
 (segment (start 118.605 95.263) (end 118.605 96.507) (width 0.25) (layer "F.Cu") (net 1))
 (segment (start 118.605 96.507) (end 118.605 97.028) (width 0.25) (layer "F.Cu") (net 1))
 (segment (start 160.954 116.504) (end 160.954 114.128) (width 0.25) (layer "F.Cu") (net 1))
 (via (at 119.126 99.06) (size 0.8) (drill 0.4) (layers "F.Cu" "B.Cu") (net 1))
 (segment (start 119.126 99.06) (end 120.358511 97.827489) (width 0.25) (layer "B.Cu") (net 1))
 (segment (start 129.069489 97.827489) (end 136.57 105.328) (width 0.25) (layer "B.Cu") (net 1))
 (segment (start 120.358511 97.827489) (end 129.069489 97.827489) (width 0.25) (layer "B.Cu") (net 1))
 (segment (start 136.57 105.328) (end 162.814 105.328) (width 0.25) (layer "B.Cu") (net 1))
 (segment (start 162.994 86.942) (end 163.068 86.868) (width 0.25) (layer "F.Cu") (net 29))
 (segment (start 155.448 86.942) (end 162.994 86.942) (width 0.25) (layer "F.Cu") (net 29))
 (segment (start 162.994 89.482) (end 163.068 89.408) (width 0.25) (layer "F.Cu") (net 30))
 (segment (start 155.448 89.482) (end 162.994 89.482) (width 0.25) (layer "F.Cu") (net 30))
 (segment (start 161.798 80.772) (end 161.730989 80.704989) (width 0.25) (layer "F.Cu") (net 33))
 (segment (start 161.730989 80.704989) (end 154.290989 80.704989) (width 0.25) (layer "F.Cu") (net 33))
 (segment (start 154.178 80.817978) (end 154.178 98.372) (width 0.25) (layer "F.Cu") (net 33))
 (segment (start 154.290989 80.704989) (end 154.178 80.817978) (width 0.25) (layer "F.Cu") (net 33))
 (segment (start 154.178 98.372) (end 155.448 99.642) (width 0.25) (layer "F.Cu") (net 33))
 (segment (start 193.04 110.231) (end 190.495 112.776) (width 0.25) (layer "F.Cu") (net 6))
 (segment (start 175.514 112.776) (end 175.514 114.128) (width 0.25) (layer "F.Cu") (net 6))
 (segment (start 190.495 112.776) (end 175.514 112.776) (width 0.25) (layer "F.Cu") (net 6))
 (segment (start 187.452 107.696) (end 177.882 107.696) (width 0.25) (layer "F.Cu") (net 34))
 (segment (start 177.882 107.696) (end 175.514 105.328) (width 0.25) (layer "F.Cu") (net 34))
 (segment (start 176.784 96.266) (end 180.086 92.964) (width 0.25) (layer "F.Cu") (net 11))
 (segment (start 169.44 96.266) (end 176.784 96.266) (width 0.25) (layer "F.Cu") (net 11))
 (segment (start 167.618 98.044) (end 180.086 98.044) (width 0.25) (layer "F.Cu") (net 12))
 (segment (start 165.84 96.266) (end 167.618 98.044) (width 0.25) (layer "F.Cu") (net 12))
 (segment (start 174.752 85.344) (end 180.086 85.344) (width 0.25) (layer "F.Cu") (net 8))
 (segment (start 173.736 86.36) (end 174.752 85.344) (width 0.25) (layer "F.Cu") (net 8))
 (segment (start 173.736 89.916) (end 177.308489 86.343511) (width 0.25) (layer "F.Cu") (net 4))
 (segment (start 180.500012 86.343511) (end 181.085511 85.758012) (width 0.25) (layer "F.Cu") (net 4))
 (segment (start 181.085511 85.758012) (end 181.085511 83.803511) (width 0.25) (layer "F.Cu") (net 4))
 (segment (start 181.085511 83.803511) (end 180.086 82.804) (width 0.25) (layer "F.Cu") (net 4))
 (segment (start 177.308489 86.343511) (end 180.500012 86.343511) (width 0.25) (layer "F.Cu") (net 4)))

